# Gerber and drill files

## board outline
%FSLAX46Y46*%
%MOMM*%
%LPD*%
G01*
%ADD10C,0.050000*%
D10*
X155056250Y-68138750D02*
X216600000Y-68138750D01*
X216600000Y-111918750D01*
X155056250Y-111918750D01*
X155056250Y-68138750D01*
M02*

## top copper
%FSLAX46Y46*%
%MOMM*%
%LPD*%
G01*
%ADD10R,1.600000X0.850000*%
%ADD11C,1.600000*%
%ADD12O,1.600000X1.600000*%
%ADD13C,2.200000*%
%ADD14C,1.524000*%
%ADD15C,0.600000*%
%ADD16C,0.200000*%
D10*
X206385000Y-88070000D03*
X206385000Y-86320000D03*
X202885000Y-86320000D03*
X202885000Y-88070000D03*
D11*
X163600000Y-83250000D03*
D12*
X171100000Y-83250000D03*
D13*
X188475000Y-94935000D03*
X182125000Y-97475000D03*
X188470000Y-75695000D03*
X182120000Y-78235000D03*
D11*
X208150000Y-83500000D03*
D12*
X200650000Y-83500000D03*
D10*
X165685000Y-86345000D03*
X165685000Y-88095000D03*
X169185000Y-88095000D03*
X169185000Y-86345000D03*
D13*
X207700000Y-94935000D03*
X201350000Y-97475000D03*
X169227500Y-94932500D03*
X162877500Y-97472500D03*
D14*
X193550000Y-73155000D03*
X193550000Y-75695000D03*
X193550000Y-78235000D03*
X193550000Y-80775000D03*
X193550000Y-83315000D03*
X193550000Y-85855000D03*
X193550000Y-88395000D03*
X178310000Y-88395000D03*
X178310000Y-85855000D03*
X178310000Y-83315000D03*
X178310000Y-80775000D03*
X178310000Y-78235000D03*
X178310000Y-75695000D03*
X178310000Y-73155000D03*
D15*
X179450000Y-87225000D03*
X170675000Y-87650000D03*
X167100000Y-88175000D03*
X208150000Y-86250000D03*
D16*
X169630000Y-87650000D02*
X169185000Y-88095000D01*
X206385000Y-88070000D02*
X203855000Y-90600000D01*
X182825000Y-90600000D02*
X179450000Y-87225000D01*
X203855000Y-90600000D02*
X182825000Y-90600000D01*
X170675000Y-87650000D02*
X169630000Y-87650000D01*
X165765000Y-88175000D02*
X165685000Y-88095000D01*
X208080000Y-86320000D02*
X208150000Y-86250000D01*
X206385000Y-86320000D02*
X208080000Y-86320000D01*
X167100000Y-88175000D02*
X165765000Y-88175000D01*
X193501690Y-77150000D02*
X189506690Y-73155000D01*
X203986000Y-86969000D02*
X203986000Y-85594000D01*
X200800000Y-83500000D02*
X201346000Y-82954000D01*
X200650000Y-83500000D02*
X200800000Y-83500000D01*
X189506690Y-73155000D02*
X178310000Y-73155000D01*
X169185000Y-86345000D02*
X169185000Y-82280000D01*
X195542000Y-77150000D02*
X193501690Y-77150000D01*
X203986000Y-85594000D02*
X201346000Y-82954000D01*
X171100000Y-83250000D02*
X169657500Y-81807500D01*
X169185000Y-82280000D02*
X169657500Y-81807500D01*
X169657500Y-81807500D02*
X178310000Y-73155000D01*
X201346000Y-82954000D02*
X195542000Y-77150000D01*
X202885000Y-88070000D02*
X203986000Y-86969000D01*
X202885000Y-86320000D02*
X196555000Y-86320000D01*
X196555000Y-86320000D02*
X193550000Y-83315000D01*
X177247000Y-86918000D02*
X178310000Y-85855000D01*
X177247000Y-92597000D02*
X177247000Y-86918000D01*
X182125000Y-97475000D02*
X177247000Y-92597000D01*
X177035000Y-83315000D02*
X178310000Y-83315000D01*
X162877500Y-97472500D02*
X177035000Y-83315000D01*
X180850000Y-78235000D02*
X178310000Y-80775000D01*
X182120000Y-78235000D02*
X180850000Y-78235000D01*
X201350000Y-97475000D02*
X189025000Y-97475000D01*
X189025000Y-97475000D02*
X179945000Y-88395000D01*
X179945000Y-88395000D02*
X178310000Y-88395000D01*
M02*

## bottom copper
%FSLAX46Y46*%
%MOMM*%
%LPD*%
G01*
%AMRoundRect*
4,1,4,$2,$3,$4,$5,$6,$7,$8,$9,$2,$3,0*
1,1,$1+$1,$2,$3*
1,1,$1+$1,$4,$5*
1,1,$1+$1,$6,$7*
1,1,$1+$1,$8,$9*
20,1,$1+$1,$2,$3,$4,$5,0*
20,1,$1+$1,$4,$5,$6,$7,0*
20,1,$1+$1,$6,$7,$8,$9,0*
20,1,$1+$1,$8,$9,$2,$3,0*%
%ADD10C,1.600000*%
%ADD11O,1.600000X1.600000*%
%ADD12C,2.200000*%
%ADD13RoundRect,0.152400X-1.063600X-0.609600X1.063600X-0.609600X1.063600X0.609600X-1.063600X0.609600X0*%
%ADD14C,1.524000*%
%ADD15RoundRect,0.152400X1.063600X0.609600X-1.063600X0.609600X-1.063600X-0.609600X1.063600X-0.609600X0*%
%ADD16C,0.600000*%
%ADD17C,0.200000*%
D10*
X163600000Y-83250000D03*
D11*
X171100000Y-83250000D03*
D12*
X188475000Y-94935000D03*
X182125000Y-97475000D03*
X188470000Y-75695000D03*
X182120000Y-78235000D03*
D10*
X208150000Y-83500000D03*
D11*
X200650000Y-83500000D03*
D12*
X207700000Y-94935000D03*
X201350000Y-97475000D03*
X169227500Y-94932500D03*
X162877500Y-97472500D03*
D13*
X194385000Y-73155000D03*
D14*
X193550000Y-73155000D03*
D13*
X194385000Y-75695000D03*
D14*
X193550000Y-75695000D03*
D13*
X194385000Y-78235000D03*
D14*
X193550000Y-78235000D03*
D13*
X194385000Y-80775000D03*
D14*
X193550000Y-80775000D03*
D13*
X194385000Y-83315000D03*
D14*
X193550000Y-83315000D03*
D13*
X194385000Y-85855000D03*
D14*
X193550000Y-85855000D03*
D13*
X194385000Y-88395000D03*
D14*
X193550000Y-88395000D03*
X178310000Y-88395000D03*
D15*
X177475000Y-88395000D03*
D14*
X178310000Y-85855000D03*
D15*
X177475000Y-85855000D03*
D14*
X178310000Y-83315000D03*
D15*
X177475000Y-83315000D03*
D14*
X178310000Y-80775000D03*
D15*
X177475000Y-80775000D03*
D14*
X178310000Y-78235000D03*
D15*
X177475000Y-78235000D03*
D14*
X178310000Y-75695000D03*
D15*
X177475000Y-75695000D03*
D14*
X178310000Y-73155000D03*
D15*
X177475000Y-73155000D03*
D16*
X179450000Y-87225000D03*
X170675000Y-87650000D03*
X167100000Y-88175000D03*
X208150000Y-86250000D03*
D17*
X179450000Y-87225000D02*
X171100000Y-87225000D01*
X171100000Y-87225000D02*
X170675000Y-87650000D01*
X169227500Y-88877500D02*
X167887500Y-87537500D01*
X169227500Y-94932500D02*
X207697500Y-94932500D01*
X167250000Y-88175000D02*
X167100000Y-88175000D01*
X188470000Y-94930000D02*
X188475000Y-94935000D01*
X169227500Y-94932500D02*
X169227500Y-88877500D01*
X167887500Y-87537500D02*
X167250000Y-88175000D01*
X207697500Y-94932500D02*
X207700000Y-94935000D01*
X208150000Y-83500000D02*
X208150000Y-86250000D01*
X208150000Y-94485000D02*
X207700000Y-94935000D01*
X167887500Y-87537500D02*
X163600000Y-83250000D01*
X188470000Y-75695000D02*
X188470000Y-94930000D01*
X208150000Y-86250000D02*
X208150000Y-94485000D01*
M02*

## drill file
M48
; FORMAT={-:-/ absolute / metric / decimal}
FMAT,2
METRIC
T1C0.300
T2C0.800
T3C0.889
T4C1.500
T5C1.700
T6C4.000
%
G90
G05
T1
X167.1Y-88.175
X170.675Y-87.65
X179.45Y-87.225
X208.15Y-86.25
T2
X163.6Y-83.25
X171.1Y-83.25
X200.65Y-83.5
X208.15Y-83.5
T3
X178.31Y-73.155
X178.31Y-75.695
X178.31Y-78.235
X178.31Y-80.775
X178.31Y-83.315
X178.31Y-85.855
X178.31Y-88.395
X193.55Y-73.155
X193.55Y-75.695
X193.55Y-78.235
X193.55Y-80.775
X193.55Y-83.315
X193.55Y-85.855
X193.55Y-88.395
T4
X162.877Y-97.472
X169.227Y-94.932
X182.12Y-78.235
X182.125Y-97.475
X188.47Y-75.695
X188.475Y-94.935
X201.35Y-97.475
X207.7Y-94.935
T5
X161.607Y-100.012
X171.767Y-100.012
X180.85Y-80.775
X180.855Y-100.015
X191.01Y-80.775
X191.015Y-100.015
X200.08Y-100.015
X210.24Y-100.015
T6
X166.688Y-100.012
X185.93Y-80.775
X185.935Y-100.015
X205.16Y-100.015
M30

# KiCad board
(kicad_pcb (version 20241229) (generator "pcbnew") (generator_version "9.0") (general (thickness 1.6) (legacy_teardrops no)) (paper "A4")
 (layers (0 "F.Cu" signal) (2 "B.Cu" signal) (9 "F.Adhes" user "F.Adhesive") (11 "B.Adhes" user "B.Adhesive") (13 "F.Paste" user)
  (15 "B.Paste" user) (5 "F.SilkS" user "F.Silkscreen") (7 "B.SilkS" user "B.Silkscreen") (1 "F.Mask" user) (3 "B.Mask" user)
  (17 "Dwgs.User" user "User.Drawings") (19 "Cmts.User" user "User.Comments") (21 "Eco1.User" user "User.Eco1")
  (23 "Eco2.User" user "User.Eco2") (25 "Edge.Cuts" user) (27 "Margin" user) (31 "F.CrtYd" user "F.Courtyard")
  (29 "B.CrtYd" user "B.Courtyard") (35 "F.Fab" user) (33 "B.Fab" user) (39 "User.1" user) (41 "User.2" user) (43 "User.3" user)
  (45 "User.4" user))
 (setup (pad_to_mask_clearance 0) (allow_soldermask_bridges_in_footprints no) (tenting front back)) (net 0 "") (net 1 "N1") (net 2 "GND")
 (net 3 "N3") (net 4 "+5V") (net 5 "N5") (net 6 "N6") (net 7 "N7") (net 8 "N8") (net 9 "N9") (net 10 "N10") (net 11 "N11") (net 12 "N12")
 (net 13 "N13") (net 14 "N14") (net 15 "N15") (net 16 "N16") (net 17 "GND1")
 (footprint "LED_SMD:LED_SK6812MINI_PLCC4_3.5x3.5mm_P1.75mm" (layer "F.Cu") (at 204.635 87.195 180)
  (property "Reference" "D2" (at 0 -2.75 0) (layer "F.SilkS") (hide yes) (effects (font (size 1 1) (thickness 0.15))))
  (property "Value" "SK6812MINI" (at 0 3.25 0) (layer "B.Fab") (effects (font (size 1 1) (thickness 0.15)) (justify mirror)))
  (pad "1" smd rect (at -1.75 -0.875 180) (size 1.6 0.85) (layers "F.Cu" "F.Mask" "F.Paste") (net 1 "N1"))
  (pad "2" smd rect (at -1.75 0.875 180) (size 1.6 0.85) (layers "F.Cu" "F.Mask" "F.Paste") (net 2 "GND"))
  (pad "3" smd rect (at 1.75 0.875 180) (size 1.6 0.85) (layers "F.Cu" "F.Mask" "F.Paste") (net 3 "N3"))
  (pad "4" smd rect (at 1.75 -0.875 180) (size 1.6 0.85) (layers "F.Cu" "F.Mask" "F.Paste") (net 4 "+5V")))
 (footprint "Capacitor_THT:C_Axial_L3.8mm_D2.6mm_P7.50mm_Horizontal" (layer "F.Cu") (at 163.6 83.25)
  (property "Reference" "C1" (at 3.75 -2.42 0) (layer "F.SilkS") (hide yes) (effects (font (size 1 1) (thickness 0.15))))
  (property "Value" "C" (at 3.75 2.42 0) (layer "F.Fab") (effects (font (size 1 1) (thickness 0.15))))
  (pad "1" thru_hole circle (at 0 0) (size 1.6 1.6) (drill 0.8) (layers "*.Cu" "*.Mask") (remove_unused_layers no) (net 2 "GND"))
  (pad "2" thru_hole oval (at 7.5 0) (size 1.6 1.6) (drill 0.8) (layers "*.Cu" "*.Mask") (remove_unused_layers no) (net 4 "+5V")))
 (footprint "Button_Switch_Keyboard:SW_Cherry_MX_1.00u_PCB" (layer "F.Cu") (at 188.475 94.935)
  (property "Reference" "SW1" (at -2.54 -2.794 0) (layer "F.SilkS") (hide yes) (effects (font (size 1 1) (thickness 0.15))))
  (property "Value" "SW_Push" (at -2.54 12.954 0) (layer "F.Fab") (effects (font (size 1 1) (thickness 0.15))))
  (pad "" np_thru_hole circle (at -7.62 5.08) (size 1.7 1.7) (drill 1.7) (layers "*.Cu" "*.Mask"))
  (pad "" np_thru_hole circle (at -2.54 5.08) (size 4 4) (drill 4) (layers "*.Cu" "*.Mask"))
  (pad "" np_thru_hole circle (at 2.54 5.08) (size 1.7 1.7) (drill 1.7) (layers "*.Cu" "*.Mask"))
  (pad "1" thru_hole circle (at 0 0) (size 2.2 2.2) (drill 1.5) (layers "*.Cu" "*.Mask") (remove_unused_layers no) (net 2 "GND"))
  (pad "2" thru_hole circle (at -6.35 2.54) (size 2.2 2.2) (drill 1.5) (layers "*.Cu" "*.Mask") (remove_unused_layers no) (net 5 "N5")))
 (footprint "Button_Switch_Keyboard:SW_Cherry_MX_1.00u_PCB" (layer "F.Cu") (at 188.47 75.695)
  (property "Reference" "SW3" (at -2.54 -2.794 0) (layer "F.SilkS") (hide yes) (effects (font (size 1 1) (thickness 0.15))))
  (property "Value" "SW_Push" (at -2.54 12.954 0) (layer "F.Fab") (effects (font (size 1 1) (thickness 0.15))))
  (pad "" np_thru_hole circle (at -7.62 5.08) (size 1.7 1.7) (drill 1.7) (layers "*.Cu" "*.Mask"))
  (pad "" np_thru_hole circle (at -2.54 5.08) (size 4 4) (drill 4) (layers "*.Cu" "*.Mask"))
  (pad "" np_thru_hole circle (at 2.54 5.08) (size 1.7 1.7) (drill 1.7) (layers "*.Cu" "*.Mask"))
  (pad "1" thru_hole circle (at 0 0) (size 2.2 2.2) (drill 1.5) (layers "*.Cu" "*.Mask") (remove_unused_layers no) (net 2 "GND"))
  (pad "2" thru_hole circle (at -6.35 2.54) (size 2.2 2.2) (drill 1.5) (layers "*.Cu" "*.Mask") (remove_unused_layers no) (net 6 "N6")))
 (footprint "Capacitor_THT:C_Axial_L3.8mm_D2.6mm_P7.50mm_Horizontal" (layer "F.Cu") (at 208.15 83.5 180)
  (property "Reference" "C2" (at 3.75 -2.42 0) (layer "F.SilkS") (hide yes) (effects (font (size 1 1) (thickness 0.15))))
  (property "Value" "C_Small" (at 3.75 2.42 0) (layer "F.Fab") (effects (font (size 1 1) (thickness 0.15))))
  (pad "1" thru_hole circle (at 0 0 180) (size 1.6 1.6) (drill 0.8) (layers "*.Cu" "*.Mask") (remove_unused_layers no) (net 2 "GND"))
  (pad "2" thru_hole oval (at 7.5 0 180) (size 1.6 1.6) (drill 0.8) (layers "*.Cu" "*.Mask") (remove_unused_layers no) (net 4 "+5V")))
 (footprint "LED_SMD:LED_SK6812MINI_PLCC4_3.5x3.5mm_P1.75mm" (layer "F.Cu") (at 167.435 87.22)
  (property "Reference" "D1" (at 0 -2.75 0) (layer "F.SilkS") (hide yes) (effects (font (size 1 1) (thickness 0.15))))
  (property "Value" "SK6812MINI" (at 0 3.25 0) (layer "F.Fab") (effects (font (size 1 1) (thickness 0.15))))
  (pad "1" smd rect (at -1.75 -0.875) (size 1.6 0.85) (layers "F.Cu" "F.Mask" "F.Paste") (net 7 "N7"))
  (pad "2" smd rect (at -1.75 0.875) (size 1.6 0.85) (layers "F.Cu" "F.Mask" "F.Paste") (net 2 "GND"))
  (pad "3" smd rect (at 1.75 0.875) (size 1.6 0.85) (layers "F.Cu" "F.Mask" "F.Paste") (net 1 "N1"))
  (pad "4" smd rect (at 1.75 -0.875) (size 1.6 0.85) (layers "F.Cu" "F.Mask" "F.Paste") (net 4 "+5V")))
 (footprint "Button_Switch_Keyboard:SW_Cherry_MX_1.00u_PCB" (layer "F.Cu") (at 207.7 94.935)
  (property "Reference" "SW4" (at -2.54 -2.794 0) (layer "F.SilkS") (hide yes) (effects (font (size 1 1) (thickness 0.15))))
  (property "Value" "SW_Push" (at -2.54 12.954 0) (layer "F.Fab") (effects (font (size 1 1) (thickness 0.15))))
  (pad "" np_thru_hole circle (at -7.62 5.08) (size 1.7 1.7) (drill 1.7) (layers "*.Cu" "*.Mask"))
  (pad "" np_thru_hole circle (at -2.54 5.08) (size 4 4) (drill 4) (layers "*.Cu" "*.Mask"))
  (pad "" np_thru_hole circle (at 2.54 5.08) (size 1.7 1.7) (drill 1.7) (layers "*.Cu" "*.Mask"))
  (pad "1" thru_hole circle (at 0 0) (size 2.2 2.2) (drill 1.5) (layers "*.Cu" "*.Mask") (remove_unused_layers no) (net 2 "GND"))
  (pad "2" thru_hole circle (at -6.35 2.54) (size 2.2 2.2) (drill 1.5) (layers "*.Cu" "*.Mask") (remove_unused_layers no) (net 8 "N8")))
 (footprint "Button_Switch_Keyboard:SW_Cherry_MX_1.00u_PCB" (layer "F.Cu") (at 169.2275 94.9325)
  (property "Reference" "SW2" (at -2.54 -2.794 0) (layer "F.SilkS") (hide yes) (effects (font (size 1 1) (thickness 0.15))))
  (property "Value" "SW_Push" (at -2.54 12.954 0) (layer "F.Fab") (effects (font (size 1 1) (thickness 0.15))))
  (pad "" np_thru_hole circle (at -7.62 5.08) (size 1.7 1.7) (drill 1.7) (layers "*.Cu" "*.Mask"))
  (pad "" np_thru_hole circle (at -2.54 5.08) (size 4 4) (drill 4) (layers "*.Cu" "*.Mask"))
  (pad "" np_thru_hole circle (at 2.54 5.08) (size 1.7 1.7) (drill 1.7) (layers "*.Cu" "*.Mask"))
  (pad "1" thru_hole circle (at 0 0) (size 2.2 2.2) (drill 1.5) (layers "*.Cu" "*.Mask") (remove_unused_layers no) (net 2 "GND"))
  (pad "2" thru_hole circle (at -6.35 2.54) (size 2.2 2.2) (drill 1.5) (layers "*.Cu" "*.Mask") (remove_unused_layers no) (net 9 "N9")))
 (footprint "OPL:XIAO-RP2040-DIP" (layer "B.Cu") (at 185.93 80.775 180)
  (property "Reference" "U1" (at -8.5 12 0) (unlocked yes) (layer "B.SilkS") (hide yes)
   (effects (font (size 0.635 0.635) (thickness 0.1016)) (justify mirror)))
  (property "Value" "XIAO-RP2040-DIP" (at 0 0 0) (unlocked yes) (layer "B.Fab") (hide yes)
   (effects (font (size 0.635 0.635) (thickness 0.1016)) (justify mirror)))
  (pad "1" smd roundrect (at -8.455 7.62) (size 2.432 1.524) (layers "B.Cu" "B.Mask") (roundrect_rratio 0.1) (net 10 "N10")
   (thermal_bridge_angle 45))
  (pad "1" thru_hole circle (at -7.62 7.62) (size 1.524 1.524) (drill 0.889) (layers "*.Cu" "*.Mask") (remove_unused_layers no)
   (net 10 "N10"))
  (pad "2" smd roundrect (at -8.455 5.08) (size 2.432 1.524) (layers "B.Cu" "B.Mask") (roundrect_rratio 0.1) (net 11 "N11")
   (thermal_bridge_angle 45))
  (pad "2" thru_hole circle (at -7.62 5.08) (size 1.524 1.524) (drill 0.889) (layers "*.Cu" "*.Mask") (remove_unused_layers no)
   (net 11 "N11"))
  (pad "3" smd roundrect (at -8.455 2.54) (size 2.432 1.524) (layers "B.Cu" "B.Mask") (roundrect_rratio 0.1) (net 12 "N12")
   (thermal_bridge_angle 45))
  (pad "3" thru_hole circle (at -7.62 2.54) (size 1.524 1.524) (drill 0.889) (layers "*.Cu" "*.Mask") (remove_unused_layers no)
   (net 12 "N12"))
  (pad "4" smd roundrect (at -8.455 0) (size 2.432 1.524) (layers "B.Cu" "B.Mask") (roundrect_rratio 0.1) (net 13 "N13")
   (thermal_bridge_angle 45))
  (pad "4" thru_hole circle (at -7.62 0) (size 1.524 1.524) (drill 0.889) (layers "*.Cu" "*.Mask") (remove_unused_layers no) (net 13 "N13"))
  (pad "5" smd roundrect (at -8.455 -2.54) (size 2.432 1.524) (layers "B.Cu" "B.Mask") (roundrect_rratio 0.1) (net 3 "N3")
   (thermal_bridge_angle 45))
  (pad "5" thru_hole circle (at -7.62 -2.54) (size 1.524 1.524) (drill 0.889) (layers "*.Cu" "*.Mask") (remove_unused_layers no)
   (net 3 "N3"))
  (pad "6" smd roundrect (at -8.455 -5.08) (size 2.432 1.524) (layers "B.Cu" "B.Mask") (roundrect_rratio 0.1) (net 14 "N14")
   (thermal_bridge_angle 45))
  (pad "6" thru_hole circle (at -7.62 -5.08) (size 1.524 1.524) (drill 0.889) (layers "*.Cu" "*.Mask") (remove_unused_layers no)
   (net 14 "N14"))
  (pad "7" smd roundrect (at -8.455 -7.62) (size 2.432 1.524) (layers "B.Cu" "B.Mask") (roundrect_rratio 0.1) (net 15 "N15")
   (thermal_bridge_angle 45))
  (pad "7" thru_hole circle (at -7.62 -7.62) (size 1.524 1.524) (drill 0.889) (layers "*.Cu" "*.Mask") (remove_unused_layers no)
   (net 15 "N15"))
  (pad "8" thru_hole circle (at 7.62 -7.62 180) (size 1.524 1.524) (drill 0.889) (layers "*.Cu" "*.Mask") (remove_unused_layers no)
   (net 8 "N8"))
  (pad "8" smd roundrect (at 8.455 -7.62 180) (size 2.432 1.524) (layers "B.Cu" "B.Mask") (roundrect_rratio 0.1) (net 8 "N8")
   (thermal_bridge_angle 45))
  (pad "9" thru_hole circle (at 7.62 -5.08 180) (size 1.524 1.524) (drill 0.889) (layers "*.Cu" "*.Mask") (remove_unused_layers no)
   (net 5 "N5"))
  (pad "9" smd roundrect (at 8.455 -5.08 180) (size 2.432 1.524) (layers "B.Cu" "B.Mask") (roundrect_rratio 0.1) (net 5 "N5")
   (thermal_bridge_angle 45))
  (pad "10" thru_hole circle (at 7.62 -2.54 180) (size 1.524 1.524) (drill 0.889) (layers "*.Cu" "*.Mask") (remove_unused_layers no)
   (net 9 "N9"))
  (pad "10" smd roundrect (at 8.455 -2.54 180) (size 2.432 1.524) (layers "B.Cu" "B.Mask") (roundrect_rratio 0.1) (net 9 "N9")
   (thermal_bridge_angle 45))
  (pad "11" thru_hole circle (at 7.62 0 180) (size 1.524 1.524) (drill 0.889) (layers "*.Cu" "*.Mask") (remove_unused_layers no)
   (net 6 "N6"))
  (pad "11" smd roundrect (at 8.455 0 180) (size 2.432 1.524) (layers "B.Cu" "B.Mask") (roundrect_rratio 0.1) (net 6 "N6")
   (thermal_bridge_angle 45))
  (pad "12" thru_hole circle (at 7.62 2.54 180) (size 1.524 1.524) (drill 0.889) (layers "*.Cu" "*.Mask") (remove_unused_layers no)
   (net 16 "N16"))
  (pad "12" smd roundrect (at 8.455 2.54 180) (size 2.432 1.524) (layers "B.Cu" "B.Mask") (roundrect_rratio 0.1) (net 16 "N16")
   (thermal_bridge_angle 45))
  (pad "13" thru_hole circle (at 7.62 5.08 180) (size 1.524 1.524) (drill 0.889) (layers "*.Cu" "*.Mask") (remove_unused_layers no)
   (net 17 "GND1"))
  (pad "13" smd roundrect (at 8.455 5.08 180) (size 2.432 1.524) (layers "B.Cu" "B.Mask") (roundrect_rratio 0.1) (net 17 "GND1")
   (thermal_bridge_angle 45))
  (pad "14" thru_hole circle (at 7.62 7.62 180) (size 1.524 1.524) (drill 0.889) (layers "*.Cu" "*.Mask") (remove_unused_layers no)
   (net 4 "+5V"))
  (pad "14" smd roundrect (at 8.455 7.62 180) (size 2.432 1.524) (layers "B.Cu" "B.Mask") (roundrect_rratio 0.1) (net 4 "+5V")
   (thermal_bridge_angle 45)))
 (gr_rect (start 155.05625 68.13875) (end 216.6 111.91875) (stroke (width 0.05) (type default)) (fill no) (layer "Edge.Cuts"))
 (segment (start 169.63 87.65) (end 169.185 88.095) (width 0.2) (layer "F.Cu") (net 1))
 (segment (start 206.385 88.07) (end 203.855 90.6) (width 0.2) (layer "F.Cu") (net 1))
 (segment (start 182.825 90.6) (end 179.45 87.225) (width 0.2) (layer "F.Cu") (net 1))
 (segment (start 203.855 90.6) (end 182.825 90.6) (width 0.2) (layer "F.Cu") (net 1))
 (segment (start 170.675 87.65) (end 169.63 87.65) (width 0.2) (layer "F.Cu") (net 1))
 (via (at 179.45 87.225) (size 0.6) (drill 0.3) (layers "F.Cu" "B.Cu") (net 1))
 (via (at 170.675 87.65) (size 0.6) (drill 0.3) (layers "F.Cu" "B.Cu") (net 1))
 (segment (start 179.45 87.225) (end 171.1 87.225) (width 0.2) (layer "B.Cu") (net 1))
 (segment (start 171.1 87.225) (end 170.675 87.65) (width 0.2) (layer "B.Cu") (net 1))
 (segment (start 165.765 88.175) (end 165.685 88.095) (width 0.2) (layer "F.Cu") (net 2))
 (segment (start 208.08 86.32) (end 208.15 86.25) (width 0.2) (layer "F.Cu") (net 2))
 (segment (start 206.385 86.32) (end 208.08 86.32) (width 0.2) (layer "F.Cu") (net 2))
 (segment (start 167.1 88.175) (end 165.765 88.175) (width 0.2) (layer "F.Cu") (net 2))
 (via (at 167.1 88.175) (size 0.6) (drill 0.3) (layers "F.Cu" "B.Cu") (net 2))
 (via (at 208.15 86.25) (size 0.6) (drill 0.3) (layers "F.Cu" "B.Cu") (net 2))
 (segment (start 169.2275 88.8775) (end 167.8875 87.5375) (width 0.2) (layer "B.Cu") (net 2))
 (segment (start 169.2275 94.9325) (end 207.6975 94.9325) (width 0.2) (layer "B.Cu") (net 2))
 (segment (start 167.25 88.175) (end 167.1 88.175) (width 0.2) (layer "B.Cu") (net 2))
 (segment (start 188.47 94.93) (end 188.475 94.935) (width 0.2) (layer "B.Cu") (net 2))
 (segment (start 169.2275 94.9325) (end 169.2275 88.8775) (width 0.2) (layer "B.Cu") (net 2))
 (segment (start 167.8875 87.5375) (end 167.25 88.175) (width 0.2) (layer "B.Cu") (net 2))
 (segment (start 207.6975 94.9325) (end 207.7 94.935) (width 0.2) (layer "B.Cu") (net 2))
 (segment (start 208.15 83.5) (end 208.15 86.25) (width 0.2) (layer "B.Cu") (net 2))
 (segment (start 208.15 94.485) (end 207.7 94.935) (width 0.2) (layer "B.Cu") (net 2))
 (segment (start 167.8875 87.5375) (end 163.6 83.25) (width 0.2) (layer "B.Cu") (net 2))
 (segment (start 188.47 75.695) (end 188.47 94.93) (width 0.2) (layer "B.Cu") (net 2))
 (segment (start 208.15 86.25) (end 208.15 94.485) (width 0.2) (layer "B.Cu") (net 2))
 (segment (start 193.50169 77.15) (end 189.50669 73.155) (width 0.2) (layer "F.Cu") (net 4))
 (segment (start 203.986 86.969) (end 203.986 85.594) (width 0.2) (layer "F.Cu") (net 4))
 (segment (start 200.8 83.5) (end 201.346 82.954) (width 0.2) (layer "F.Cu") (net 4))
 (segment (start 200.65 83.5) (end 200.8 83.5) (width 0.2) (layer "F.Cu") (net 4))
 (segment (start 189.50669 73.155) (end 178.31 73.155) (width 0.2) (layer "F.Cu") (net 4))
 (segment (start 169.185 86.345) (end 169.185 82.28) (width 0.2) (layer "F.Cu") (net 4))
 (segment (start 195.542 77.15) (end 193.50169 77.15) (width 0.2) (layer "F.Cu") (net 4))
 (segment (start 203.986 85.594) (end 201.346 82.954) (width 0.2) (layer "F.Cu") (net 4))
 (segment (start 171.1 83.25) (end 169.6575 81.8075) (width 0.2) (layer "F.Cu") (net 4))
 (segment (start 169.185 82.28) (end 169.6575 81.8075) (width 0.2) (layer "F.Cu") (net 4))
 (segment (start 169.6575 81.8075) (end 178.31 73.155) (width 0.2) (layer "F.Cu") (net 4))
 (segment (start 201.346 82.954) (end 195.542 77.15) (width 0.2) (layer "F.Cu") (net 4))
 (segment (start 202.885 88.07) (end 203.986 86.969) (width 0.2) (layer "F.Cu") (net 4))
 (segment (start 202.885 86.32) (end 196.555 86.32) (width 0.2) (layer "F.Cu") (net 3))
 (segment (start 196.555 86.32) (end 193.55 83.315) (width 0.2) (layer "F.Cu") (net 3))
 (segment (start 177.247 86.918) (end 178.31 85.855) (width 0.2) (layer "F.Cu") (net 5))
 (segment (start 177.247 92.597) (end 177.247 86.918) (width 0.2) (layer "F.Cu") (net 5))
 (segment (start 182.125 97.475) (end 177.247 92.597) (width 0.2) (layer "F.Cu") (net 5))
 (segment (start 177.035 83.315) (end 178.31 83.315) (width 0.2) (layer "F.Cu") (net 9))
 (segment (start 162.8775 97.4725) (end 177.035 83.315) (width 0.2) (layer "F.Cu") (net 9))
 (segment (start 180.85 78.235) (end 178.31 80.775) (width 0.2) (layer "F.Cu") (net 6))
 (segment (start 182.12 78.235) (end 180.85 78.235) (width 0.2) (layer "F.Cu") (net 6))
 (segment (start 201.35 97.475) (end 189.025 97.475) (width 0.2) (layer "F.Cu") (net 8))
 (segment (start 189.025 97.475) (end 179.945 88.395) (width 0.2) (layer "F.Cu") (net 8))
 (segment (start 179.945 88.395) (end 178.31 88.395) (width 0.2) (layer "F.Cu") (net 8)))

